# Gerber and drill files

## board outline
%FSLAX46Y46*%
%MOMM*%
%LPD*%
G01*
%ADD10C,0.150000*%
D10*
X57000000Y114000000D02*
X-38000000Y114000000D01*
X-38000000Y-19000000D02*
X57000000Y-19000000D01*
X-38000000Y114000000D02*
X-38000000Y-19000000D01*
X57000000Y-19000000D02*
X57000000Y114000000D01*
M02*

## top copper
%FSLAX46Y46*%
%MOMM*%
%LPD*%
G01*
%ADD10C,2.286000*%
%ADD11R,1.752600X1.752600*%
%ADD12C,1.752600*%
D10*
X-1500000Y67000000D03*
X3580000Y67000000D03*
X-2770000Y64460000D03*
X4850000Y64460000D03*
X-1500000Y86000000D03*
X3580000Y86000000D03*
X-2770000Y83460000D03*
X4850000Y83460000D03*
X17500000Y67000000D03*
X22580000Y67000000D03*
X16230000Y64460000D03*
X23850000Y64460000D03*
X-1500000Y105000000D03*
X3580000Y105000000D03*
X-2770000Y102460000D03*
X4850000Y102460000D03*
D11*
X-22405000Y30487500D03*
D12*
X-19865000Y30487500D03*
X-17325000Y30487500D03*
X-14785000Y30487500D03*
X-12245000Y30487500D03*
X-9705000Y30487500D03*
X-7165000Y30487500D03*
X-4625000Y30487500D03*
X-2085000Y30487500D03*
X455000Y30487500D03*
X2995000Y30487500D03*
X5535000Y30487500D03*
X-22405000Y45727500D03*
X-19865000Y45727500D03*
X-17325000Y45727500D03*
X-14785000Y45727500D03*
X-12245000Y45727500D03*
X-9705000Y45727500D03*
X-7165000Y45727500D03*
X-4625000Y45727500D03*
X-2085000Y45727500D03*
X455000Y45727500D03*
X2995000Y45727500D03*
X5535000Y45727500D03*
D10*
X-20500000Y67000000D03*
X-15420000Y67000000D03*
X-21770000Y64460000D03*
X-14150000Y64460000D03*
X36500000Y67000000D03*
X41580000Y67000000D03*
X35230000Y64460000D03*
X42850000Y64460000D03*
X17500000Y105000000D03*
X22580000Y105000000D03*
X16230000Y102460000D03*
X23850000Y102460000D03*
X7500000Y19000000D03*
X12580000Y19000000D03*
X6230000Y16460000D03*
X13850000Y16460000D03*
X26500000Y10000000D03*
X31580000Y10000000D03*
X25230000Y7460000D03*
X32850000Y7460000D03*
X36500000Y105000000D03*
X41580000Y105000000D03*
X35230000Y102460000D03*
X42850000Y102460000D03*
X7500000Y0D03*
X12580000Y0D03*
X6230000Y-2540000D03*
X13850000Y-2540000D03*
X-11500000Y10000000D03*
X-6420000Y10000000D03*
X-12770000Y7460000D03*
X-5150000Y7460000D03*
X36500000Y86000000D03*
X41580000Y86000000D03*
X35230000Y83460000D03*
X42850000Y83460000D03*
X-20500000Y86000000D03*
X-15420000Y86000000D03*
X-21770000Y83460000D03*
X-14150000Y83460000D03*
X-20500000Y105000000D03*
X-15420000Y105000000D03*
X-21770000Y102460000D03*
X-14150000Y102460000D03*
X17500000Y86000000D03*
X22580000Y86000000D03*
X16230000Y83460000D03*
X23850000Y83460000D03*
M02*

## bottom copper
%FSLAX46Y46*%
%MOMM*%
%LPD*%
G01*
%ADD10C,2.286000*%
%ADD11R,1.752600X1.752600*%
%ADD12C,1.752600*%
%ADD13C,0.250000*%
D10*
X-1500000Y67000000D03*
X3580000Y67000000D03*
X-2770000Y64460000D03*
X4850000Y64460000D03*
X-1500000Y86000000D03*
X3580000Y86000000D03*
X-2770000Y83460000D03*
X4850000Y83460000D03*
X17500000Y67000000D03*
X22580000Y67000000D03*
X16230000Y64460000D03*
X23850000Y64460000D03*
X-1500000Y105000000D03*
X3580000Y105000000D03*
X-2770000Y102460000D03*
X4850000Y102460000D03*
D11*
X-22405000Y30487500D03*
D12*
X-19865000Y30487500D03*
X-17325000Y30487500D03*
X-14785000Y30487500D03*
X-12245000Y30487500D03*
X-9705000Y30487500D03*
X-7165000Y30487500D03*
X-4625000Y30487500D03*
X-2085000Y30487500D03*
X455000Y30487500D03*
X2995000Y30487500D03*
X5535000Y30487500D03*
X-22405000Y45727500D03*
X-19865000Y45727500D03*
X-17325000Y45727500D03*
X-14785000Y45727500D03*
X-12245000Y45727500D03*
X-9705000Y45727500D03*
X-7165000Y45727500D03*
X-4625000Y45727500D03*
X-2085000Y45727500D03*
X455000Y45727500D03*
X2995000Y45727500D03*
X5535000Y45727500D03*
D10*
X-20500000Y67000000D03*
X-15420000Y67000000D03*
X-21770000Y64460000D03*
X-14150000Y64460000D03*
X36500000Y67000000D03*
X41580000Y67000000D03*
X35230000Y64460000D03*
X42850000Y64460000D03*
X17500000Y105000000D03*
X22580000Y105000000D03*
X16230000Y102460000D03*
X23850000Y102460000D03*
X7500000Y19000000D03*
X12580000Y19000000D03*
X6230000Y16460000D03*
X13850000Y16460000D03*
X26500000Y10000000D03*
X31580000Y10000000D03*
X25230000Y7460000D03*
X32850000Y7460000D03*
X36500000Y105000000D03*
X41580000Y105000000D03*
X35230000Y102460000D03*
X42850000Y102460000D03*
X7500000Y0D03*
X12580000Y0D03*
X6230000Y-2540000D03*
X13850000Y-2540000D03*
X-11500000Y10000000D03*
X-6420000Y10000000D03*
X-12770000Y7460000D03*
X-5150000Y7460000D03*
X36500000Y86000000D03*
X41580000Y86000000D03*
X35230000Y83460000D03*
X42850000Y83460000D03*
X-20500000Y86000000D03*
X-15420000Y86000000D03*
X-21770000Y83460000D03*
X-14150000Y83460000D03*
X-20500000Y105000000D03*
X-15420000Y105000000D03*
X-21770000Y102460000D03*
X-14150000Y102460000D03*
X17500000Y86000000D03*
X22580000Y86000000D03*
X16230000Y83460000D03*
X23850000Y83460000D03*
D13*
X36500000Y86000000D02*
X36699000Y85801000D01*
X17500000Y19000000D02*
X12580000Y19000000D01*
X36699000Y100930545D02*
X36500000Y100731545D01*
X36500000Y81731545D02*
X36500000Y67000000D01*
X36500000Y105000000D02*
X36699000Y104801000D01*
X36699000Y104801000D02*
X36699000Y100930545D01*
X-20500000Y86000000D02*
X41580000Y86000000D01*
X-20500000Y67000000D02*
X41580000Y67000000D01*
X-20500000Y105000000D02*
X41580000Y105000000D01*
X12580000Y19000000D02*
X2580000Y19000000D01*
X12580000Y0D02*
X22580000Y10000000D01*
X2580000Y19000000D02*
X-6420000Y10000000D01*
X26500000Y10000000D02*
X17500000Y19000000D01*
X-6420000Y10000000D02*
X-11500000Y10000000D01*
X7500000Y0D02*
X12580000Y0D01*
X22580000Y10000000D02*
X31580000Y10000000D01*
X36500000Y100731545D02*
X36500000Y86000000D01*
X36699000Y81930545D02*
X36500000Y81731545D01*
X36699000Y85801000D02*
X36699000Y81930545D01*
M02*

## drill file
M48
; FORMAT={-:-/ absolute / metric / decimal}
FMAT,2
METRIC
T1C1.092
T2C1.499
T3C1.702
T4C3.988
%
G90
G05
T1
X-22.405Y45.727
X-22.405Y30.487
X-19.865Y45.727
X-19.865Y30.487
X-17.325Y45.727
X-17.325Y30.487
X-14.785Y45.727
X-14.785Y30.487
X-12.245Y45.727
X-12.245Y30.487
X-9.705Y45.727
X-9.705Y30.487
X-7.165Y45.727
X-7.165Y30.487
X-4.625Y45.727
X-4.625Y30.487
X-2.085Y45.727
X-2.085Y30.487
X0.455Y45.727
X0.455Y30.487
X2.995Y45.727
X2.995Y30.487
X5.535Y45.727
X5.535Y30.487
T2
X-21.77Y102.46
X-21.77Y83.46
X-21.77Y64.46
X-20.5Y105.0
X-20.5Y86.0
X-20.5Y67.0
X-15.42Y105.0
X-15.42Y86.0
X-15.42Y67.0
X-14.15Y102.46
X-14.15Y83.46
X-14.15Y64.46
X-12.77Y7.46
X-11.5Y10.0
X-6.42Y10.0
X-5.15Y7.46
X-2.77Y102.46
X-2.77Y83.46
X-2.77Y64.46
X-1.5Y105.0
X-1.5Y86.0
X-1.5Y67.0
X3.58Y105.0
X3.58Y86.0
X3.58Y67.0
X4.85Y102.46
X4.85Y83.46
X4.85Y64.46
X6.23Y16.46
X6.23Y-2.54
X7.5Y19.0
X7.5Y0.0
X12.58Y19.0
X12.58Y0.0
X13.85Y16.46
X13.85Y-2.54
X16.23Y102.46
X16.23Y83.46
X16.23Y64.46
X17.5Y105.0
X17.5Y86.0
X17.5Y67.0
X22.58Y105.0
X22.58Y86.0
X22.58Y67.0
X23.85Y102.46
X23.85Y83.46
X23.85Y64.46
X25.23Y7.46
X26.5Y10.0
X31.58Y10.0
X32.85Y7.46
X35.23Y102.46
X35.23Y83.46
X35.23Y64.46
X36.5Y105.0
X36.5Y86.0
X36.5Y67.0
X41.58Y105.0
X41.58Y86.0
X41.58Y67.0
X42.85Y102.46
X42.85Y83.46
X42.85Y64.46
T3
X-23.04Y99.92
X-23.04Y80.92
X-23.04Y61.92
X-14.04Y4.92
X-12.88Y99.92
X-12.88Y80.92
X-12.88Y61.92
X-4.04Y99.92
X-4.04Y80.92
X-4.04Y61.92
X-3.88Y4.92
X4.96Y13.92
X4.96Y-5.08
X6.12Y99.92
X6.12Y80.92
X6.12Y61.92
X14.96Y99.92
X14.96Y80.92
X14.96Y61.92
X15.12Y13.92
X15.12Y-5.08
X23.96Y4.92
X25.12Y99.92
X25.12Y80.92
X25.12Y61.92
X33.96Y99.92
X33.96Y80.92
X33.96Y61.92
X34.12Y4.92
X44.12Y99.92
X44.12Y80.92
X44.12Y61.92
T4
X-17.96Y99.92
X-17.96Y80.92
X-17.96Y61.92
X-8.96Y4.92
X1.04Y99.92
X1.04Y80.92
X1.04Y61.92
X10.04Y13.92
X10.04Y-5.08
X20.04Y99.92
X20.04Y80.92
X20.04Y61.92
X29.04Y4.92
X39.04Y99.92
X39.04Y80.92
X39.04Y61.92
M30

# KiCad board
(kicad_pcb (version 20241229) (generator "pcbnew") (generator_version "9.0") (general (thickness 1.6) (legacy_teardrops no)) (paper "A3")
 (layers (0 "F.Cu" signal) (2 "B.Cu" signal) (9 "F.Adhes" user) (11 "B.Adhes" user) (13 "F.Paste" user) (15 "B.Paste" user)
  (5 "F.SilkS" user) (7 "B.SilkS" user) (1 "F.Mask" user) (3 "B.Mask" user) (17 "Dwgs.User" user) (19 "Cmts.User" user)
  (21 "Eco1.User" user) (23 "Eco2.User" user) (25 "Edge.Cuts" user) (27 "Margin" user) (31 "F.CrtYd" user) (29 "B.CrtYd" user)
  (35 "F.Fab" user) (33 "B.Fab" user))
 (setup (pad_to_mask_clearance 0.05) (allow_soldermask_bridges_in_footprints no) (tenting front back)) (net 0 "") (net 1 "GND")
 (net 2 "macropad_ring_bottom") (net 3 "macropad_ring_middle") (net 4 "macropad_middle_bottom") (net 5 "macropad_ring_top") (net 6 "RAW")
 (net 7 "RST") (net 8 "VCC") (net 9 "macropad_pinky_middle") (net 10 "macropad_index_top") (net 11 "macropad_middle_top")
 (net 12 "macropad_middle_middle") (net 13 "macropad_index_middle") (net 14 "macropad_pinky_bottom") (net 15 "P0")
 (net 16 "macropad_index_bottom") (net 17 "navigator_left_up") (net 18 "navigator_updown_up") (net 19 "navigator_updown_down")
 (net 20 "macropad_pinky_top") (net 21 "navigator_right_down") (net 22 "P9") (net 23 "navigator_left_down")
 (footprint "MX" (layer "F.Cu") (at 1.04 -61.92)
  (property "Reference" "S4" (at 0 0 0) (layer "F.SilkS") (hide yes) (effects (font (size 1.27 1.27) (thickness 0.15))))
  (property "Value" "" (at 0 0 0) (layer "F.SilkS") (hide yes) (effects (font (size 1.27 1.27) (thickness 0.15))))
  (pad "" np_thru_hole circle (at -5.08 0) (size 1.7018 1.7018) (drill 1.7018) (layers "*.Cu" "*.Mask"))
  (pad "" np_thru_hole circle (at 0 0) (size 3.9878 3.9878) (drill 3.9878) (layers "*.Cu" "*.Mask"))
  (pad "" np_thru_hole circle (at 5.08 0) (size 1.7018 1.7018) (drill 1.7018) (layers "*.Cu" "*.Mask"))
  (pad "1" thru_hole circle (at -2.54 -5.08) (size 2.286 2.286) (drill 1.4986) (layers "*.Cu" "*.Mask") (remove_unused_layers no)
   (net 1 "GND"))
  (pad "1" thru_hole circle (at 2.54 -5.08) (size 2.286 2.286) (drill 1.4986) (layers "*.Cu" "*.Mask") (remove_unused_layers no)
   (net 1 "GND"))
  (pad "2" thru_hole circle (at -3.81 -2.54) (size 2.286 2.286) (drill 1.4986) (layers "*.Cu" "*.Mask") (remove_unused_layers no)
   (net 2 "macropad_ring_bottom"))
  (pad "2" thru_hole circle (at 3.81 -2.54) (size 2.286 2.286) (drill 1.4986) (layers "*.Cu" "*.Mask") (remove_unused_layers no)
   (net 2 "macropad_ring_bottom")))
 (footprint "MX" (layer "F.Cu") (at 1.04 -80.92)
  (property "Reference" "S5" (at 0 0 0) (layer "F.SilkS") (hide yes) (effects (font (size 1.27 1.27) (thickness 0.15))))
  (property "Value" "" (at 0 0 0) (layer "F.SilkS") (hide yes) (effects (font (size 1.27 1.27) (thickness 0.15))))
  (pad "" np_thru_hole circle (at -5.08 0) (size 1.7018 1.7018) (drill 1.7018) (layers "*.Cu" "*.Mask"))
  (pad "" np_thru_hole circle (at 0 0) (size 3.9878 3.9878) (drill 3.9878) (layers "*.Cu" "*.Mask"))
  (pad "" np_thru_hole circle (at 5.08 0) (size 1.7018 1.7018) (drill 1.7018) (layers "*.Cu" "*.Mask"))
  (pad "1" thru_hole circle (at -2.54 -5.08) (size 2.286 2.286) (drill 1.4986) (layers "*.Cu" "*.Mask") (remove_unused_layers no)
   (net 1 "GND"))
  (pad "1" thru_hole circle (at 2.54 -5.08) (size 2.286 2.286) (drill 1.4986) (layers "*.Cu" "*.Mask") (remove_unused_layers no)
   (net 1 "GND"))
  (pad "2" thru_hole circle (at -3.81 -2.54) (size 2.286 2.286) (drill 1.4986) (layers "*.Cu" "*.Mask") (remove_unused_layers no)
   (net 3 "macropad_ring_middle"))
  (pad "2" thru_hole circle (at 3.81 -2.54) (size 2.286 2.286) (drill 1.4986) (layers "*.Cu" "*.Mask") (remove_unused_layers no)
   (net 3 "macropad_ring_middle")))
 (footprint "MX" (layer "F.Cu") (at 20.04 -61.92)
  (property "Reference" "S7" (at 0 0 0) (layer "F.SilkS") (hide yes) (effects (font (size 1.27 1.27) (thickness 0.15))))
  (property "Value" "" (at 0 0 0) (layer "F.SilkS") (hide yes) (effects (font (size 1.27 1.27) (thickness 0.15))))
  (pad "" np_thru_hole circle (at -5.08 0) (size 1.7018 1.7018) (drill 1.7018) (layers "*.Cu" "*.Mask"))
  (pad "" np_thru_hole circle (at 0 0) (size 3.9878 3.9878) (drill 3.9878) (layers "*.Cu" "*.Mask"))
  (pad "" np_thru_hole circle (at 5.08 0) (size 1.7018 1.7018) (drill 1.7018) (layers "*.Cu" "*.Mask"))
  (pad "1" thru_hole circle (at -2.54 -5.08) (size 2.286 2.286) (drill 1.4986) (layers "*.Cu" "*.Mask") (remove_unused_layers no)
   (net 1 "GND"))
  (pad "1" thru_hole circle (at 2.54 -5.08) (size 2.286 2.286) (drill 1.4986) (layers "*.Cu" "*.Mask") (remove_unused_layers no)
   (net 1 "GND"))
  (pad "2" thru_hole circle (at -3.81 -2.54) (size 2.286 2.286) (drill 1.4986) (layers "*.Cu" "*.Mask") (remove_unused_layers no)
   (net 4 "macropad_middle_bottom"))
  (pad "2" thru_hole circle (at 3.81 -2.54) (size 2.286 2.286) (drill 1.4986) (layers "*.Cu" "*.Mask") (remove_unused_layers no)
   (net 4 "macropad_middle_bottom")))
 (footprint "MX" (layer "F.Cu") (at 1.04 -99.92)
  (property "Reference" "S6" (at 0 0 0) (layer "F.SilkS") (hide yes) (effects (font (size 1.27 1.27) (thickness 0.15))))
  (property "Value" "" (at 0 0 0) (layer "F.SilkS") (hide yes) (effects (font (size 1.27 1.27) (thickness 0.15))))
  (pad "" np_thru_hole circle (at -5.08 0) (size 1.7018 1.7018) (drill 1.7018) (layers "*.Cu" "*.Mask"))
  (pad "" np_thru_hole circle (at 0 0) (size 3.9878 3.9878) (drill 3.9878) (layers "*.Cu" "*.Mask"))
  (pad "" np_thru_hole circle (at 5.08 0) (size 1.7018 1.7018) (drill 1.7018) (layers "*.Cu" "*.Mask"))
  (pad "1" thru_hole circle (at -2.54 -5.08) (size 2.286 2.286) (drill 1.4986) (layers "*.Cu" "*.Mask") (remove_unused_layers no)
   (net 1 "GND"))
  (pad "1" thru_hole circle (at 2.54 -5.08) (size 2.286 2.286) (drill 1.4986) (layers "*.Cu" "*.Mask") (remove_unused_layers no)
   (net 1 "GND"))
  (pad "2" thru_hole circle (at -3.81 -2.54) (size 2.286 2.286) (drill 1.4986) (layers "*.Cu" "*.Mask") (remove_unused_layers no)
   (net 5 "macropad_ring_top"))
  (pad "2" thru_hole circle (at 3.81 -2.54) (size 2.286 2.286) (drill 1.4986) (layers "*.Cu" "*.Mask") (remove_unused_layers no)
   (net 5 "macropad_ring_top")))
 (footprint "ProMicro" (layer "F.Cu") (at -8.435 -38.1075)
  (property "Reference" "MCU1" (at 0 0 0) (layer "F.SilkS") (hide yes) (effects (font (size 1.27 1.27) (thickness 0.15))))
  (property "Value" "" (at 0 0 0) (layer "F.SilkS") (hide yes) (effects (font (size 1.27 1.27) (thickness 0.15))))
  (pad "1" thru_hole rect (at -13.97 7.62) (size 1.7526 1.7526) (drill 1.0922) (layers "*.Cu" "*.SilkS" "*.Mask") (remove_unused_layers no)
   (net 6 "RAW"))
  (pad "2" thru_hole circle (at -11.43 7.62) (size 1.7526 1.7526) (drill 1.0922) (layers "*.Cu" "*.SilkS" "*.Mask")
   (remove_unused_layers no) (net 1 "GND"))
  (pad "3" thru_hole circle (at -8.89 7.62) (size 1.7526 1.7526) (drill 1.0922) (layers "*.Cu" "*.SilkS" "*.Mask") (remove_unused_layers no)
   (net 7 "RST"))
  (pad "4" thru_hole circle (at -6.35 7.62) (size 1.7526 1.7526) (drill 1.0922) (layers "*.Cu" "*.SilkS" "*.Mask") (remove_unused_layers no)
   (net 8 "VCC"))
  (pad "5" thru_hole circle (at -3.81 7.62) (size 1.7526 1.7526) (drill 1.0922) (layers "*.Cu" "*.SilkS" "*.Mask") (remove_unused_layers no)
   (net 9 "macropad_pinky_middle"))
  (pad "6" thru_hole circle (at -1.27 7.62) (size 1.7526 1.7526) (drill 1.0922) (layers "*.Cu" "*.SilkS" "*.Mask") (remove_unused_layers no)
   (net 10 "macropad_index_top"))
  (pad "7" thru_hole circle (at 1.27 7.62) (size 1.7526 1.7526) (drill 1.0922) (layers "*.Cu" "*.SilkS" "*.Mask") (remove_unused_layers no)
   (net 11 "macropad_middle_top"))
  (pad "8" thru_hole circle (at 3.81 7.62) (size 1.7526 1.7526) (drill 1.0922) (layers "*.Cu" "*.SilkS" "*.Mask") (remove_unused_layers no)
   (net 5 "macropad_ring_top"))
  (pad "9" thru_hole circle (at 6.35 7.62) (size 1.7526 1.7526) (drill 1.0922) (layers "*.Cu" "*.SilkS" "*.Mask") (remove_unused_layers no)
   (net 3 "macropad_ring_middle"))
  (pad "10" thru_hole circle (at 8.89 7.62) (size 1.7526 1.7526) (drill 1.0922) (layers "*.Cu" "*.SilkS" "*.Mask") (remove_unused_layers no)
   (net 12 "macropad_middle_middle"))
  (pad "11" thru_hole circle (at 11.43 7.62) (size 1.7526 1.7526) (drill 1.0922) (layers "*.Cu" "*.SilkS" "*.Mask")
   (remove_unused_layers no) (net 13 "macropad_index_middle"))
  (pad "12" thru_hole circle (at 13.97 7.62) (size 1.7526 1.7526) (drill 1.0922) (layers "*.Cu" "*.SilkS" "*.Mask")
   (remove_unused_layers no) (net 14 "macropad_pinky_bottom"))
  (pad "13" thru_hole circle (at -13.97 -7.62) (size 1.7526 1.7526) (drill 1.0922) (layers "*.Cu" "*.SilkS" "*.Mask")
   (remove_unused_layers no) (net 2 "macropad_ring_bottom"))
  (pad "14" thru_hole circle (at -11.43 -7.62) (size 1.7526 1.7526) (drill 1.0922) (layers "*.Cu" "*.SilkS" "*.Mask")
   (remove_unused_layers no) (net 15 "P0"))
  (pad "15" thru_hole circle (at -8.89 -7.62) (size 1.7526 1.7526) (drill 1.0922) (layers "*.Cu" "*.SilkS" "*.Mask")
   (remove_unused_layers no) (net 1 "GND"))
  (pad "16" thru_hole circle (at -6.35 -7.62) (size 1.7526 1.7526) (drill 1.0922) (layers "*.Cu" "*.SilkS" "*.Mask")
   (remove_unused_layers no) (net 1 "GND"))
  (pad "17" thru_hole circle (at -3.81 -7.62) (size 1.7526 1.7526) (drill 1.0922) (layers "*.Cu" "*.SilkS" "*.Mask")
   (remove_unused_layers no) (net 4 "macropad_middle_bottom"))
  (pad "18" thru_hole circle (at -1.27 -7.62) (size 1.7526 1.7526) (drill 1.0922) (layers "*.Cu" "*.SilkS" "*.Mask")
   (remove_unused_layers no) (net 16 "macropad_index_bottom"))
  (pad "19" thru_hole circle (at 1.27 -7.62) (size 1.7526 1.7526) (drill 1.0922) (layers "*.Cu" "*.SilkS" "*.Mask")
   (remove_unused_layers no) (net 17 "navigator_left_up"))
  (pad "20" thru_hole circle (at 3.81 -7.62) (size 1.7526 1.7526) (drill 1.0922) (layers "*.Cu" "*.SilkS" "*.Mask")
   (remove_unused_layers no) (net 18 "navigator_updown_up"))
  (pad "21" thru_hole circle (at 6.35 -7.62) (size 1.7526 1.7526) (drill 1.0922) (layers "*.Cu" "*.SilkS" "*.Mask")
   (remove_unused_layers no) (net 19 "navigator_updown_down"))
  (pad "22" thru_hole circle (at 8.89 -7.62) (size 1.7526 1.7526) (drill 1.0922) (layers "*.Cu" "*.SilkS" "*.Mask")
   (remove_unused_layers no) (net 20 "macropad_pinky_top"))
  (pad "23" thru_hole circle (at 11.43 -7.62) (size 1.7526 1.7526) (drill 1.0922) (layers "*.Cu" "*.SilkS" "*.Mask")
   (remove_unused_layers no) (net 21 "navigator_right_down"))
  (pad "24" thru_hole circle (at 13.97 -7.62) (size 1.7526 1.7526) (drill 1.0922) (layers "*.Cu" "*.SilkS" "*.Mask")
   (remove_unused_layers no) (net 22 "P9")))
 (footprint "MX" (layer "F.Cu") (at -17.96 -61.92)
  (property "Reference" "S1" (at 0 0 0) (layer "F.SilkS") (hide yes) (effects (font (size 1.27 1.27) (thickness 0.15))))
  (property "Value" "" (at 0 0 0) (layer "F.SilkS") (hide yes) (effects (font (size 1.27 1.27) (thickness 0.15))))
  (pad "" np_thru_hole circle (at -5.08 0) (size 1.7018 1.7018) (drill 1.7018) (layers "*.Cu" "*.Mask"))
  (pad "" np_thru_hole circle (at 0 0) (size 3.9878 3.9878) (drill 3.9878) (layers "*.Cu" "*.Mask"))
  (pad "" np_thru_hole circle (at 5.08 0) (size 1.7018 1.7018) (drill 1.7018) (layers "*.Cu" "*.Mask"))
  (pad "1" thru_hole circle (at -2.54 -5.08) (size 2.286 2.286) (drill 1.4986) (layers "*.Cu" "*.Mask") (remove_unused_layers no)
   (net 1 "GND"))
  (pad "1" thru_hole circle (at 2.54 -5.08) (size 2.286 2.286) (drill 1.4986) (layers "*.Cu" "*.Mask") (remove_unused_layers no)
   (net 1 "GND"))
  (pad "2" thru_hole circle (at -3.81 -2.54) (size 2.286 2.286) (drill 1.4986) (layers "*.Cu" "*.Mask") (remove_unused_layers no)
   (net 14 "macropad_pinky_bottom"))
  (pad "2" thru_hole circle (at 3.81 -2.54) (size 2.286 2.286) (drill 1.4986) (layers "*.Cu" "*.Mask") (remove_unused_layers no)
   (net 14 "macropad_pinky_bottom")))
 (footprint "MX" (layer "F.Cu") (at 39.04 -61.92)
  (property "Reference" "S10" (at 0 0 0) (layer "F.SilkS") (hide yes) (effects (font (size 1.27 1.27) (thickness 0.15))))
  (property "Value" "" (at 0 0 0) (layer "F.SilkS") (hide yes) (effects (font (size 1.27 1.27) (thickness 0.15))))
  (pad "" np_thru_hole circle (at -5.08 0) (size 1.7018 1.7018) (drill 1.7018) (layers "*.Cu" "*.Mask"))
  (pad "" np_thru_hole circle (at 0 0) (size 3.9878 3.9878) (drill 3.9878) (layers "*.Cu" "*.Mask"))
  (pad "" np_thru_hole circle (at 5.08 0) (size 1.7018 1.7018) (drill 1.7018) (layers "*.Cu" "*.Mask"))
  (pad "1" thru_hole circle (at -2.54 -5.08) (size 2.286 2.286) (drill 1.4986) (layers "*.Cu" "*.Mask") (remove_unused_layers no)
   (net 1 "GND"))
  (pad "1" thru_hole circle (at 2.54 -5.08) (size 2.286 2.286) (drill 1.4986) (layers "*.Cu" "*.Mask") (remove_unused_layers no)
   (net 1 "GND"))
  (pad "2" thru_hole circle (at -3.81 -2.54) (size 2.286 2.286) (drill 1.4986) (layers "*.Cu" "*.Mask") (remove_unused_layers no)
   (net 16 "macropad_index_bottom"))
  (pad "2" thru_hole circle (at 3.81 -2.54) (size 2.286 2.286) (drill 1.4986) (layers "*.Cu" "*.Mask") (remove_unused_layers no)
   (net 16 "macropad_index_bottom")))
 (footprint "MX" (layer "F.Cu") (at 20.04 -99.92)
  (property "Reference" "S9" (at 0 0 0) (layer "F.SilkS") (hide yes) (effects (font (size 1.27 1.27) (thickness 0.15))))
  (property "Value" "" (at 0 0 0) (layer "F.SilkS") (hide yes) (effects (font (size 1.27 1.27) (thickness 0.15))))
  (pad "" np_thru_hole circle (at -5.08 0) (size 1.7018 1.7018) (drill 1.7018) (layers "*.Cu" "*.Mask"))
  (pad "" np_thru_hole circle (at 0 0) (size 3.9878 3.9878) (drill 3.9878) (layers "*.Cu" "*.Mask"))
  (pad "" np_thru_hole circle (at 5.08 0) (size 1.7018 1.7018) (drill 1.7018) (layers "*.Cu" "*.Mask"))
  (pad "1" thru_hole circle (at -2.54 -5.08) (size 2.286 2.286) (drill 1.4986) (layers "*.Cu" "*.Mask") (remove_unused_layers no)
   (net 1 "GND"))
  (pad "1" thru_hole circle (at 2.54 -5.08) (size 2.286 2.286) (drill 1.4986) (layers "*.Cu" "*.Mask") (remove_unused_layers no)
   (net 1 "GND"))
  (pad "2" thru_hole circle (at -3.81 -2.54) (size 2.286 2.286) (drill 1.4986) (layers "*.Cu" "*.Mask") (remove_unused_layers no)
   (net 11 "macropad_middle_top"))
  (pad "2" thru_hole circle (at 3.81 -2.54) (size 2.286 2.286) (drill 1.4986) (layers "*.Cu" "*.Mask") (remove_unused_layers no)
   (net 11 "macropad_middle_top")))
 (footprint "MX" (layer "F.Cu") (at 10.04 -13.92)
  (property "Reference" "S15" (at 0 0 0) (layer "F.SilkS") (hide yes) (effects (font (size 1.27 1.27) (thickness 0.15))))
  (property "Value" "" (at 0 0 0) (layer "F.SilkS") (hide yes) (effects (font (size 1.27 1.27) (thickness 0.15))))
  (pad "" np_thru_hole circle (at -5.08 0) (size 1.7018 1.7018) (drill 1.7018) (layers "*.Cu" "*.Mask"))
  (pad "" np_thru_hole circle (at 0 0) (size 3.9878 3.9878) (drill 3.9878) (layers "*.Cu" "*.Mask"))
  (pad "" np_thru_hole circle (at 5.08 0) (size 1.7018 1.7018) (drill 1.7018) (layers "*.Cu" "*.Mask"))
  (pad "1" thru_hole circle (at -2.54 -5.08) (size 2.286 2.286) (drill 1.4986) (layers "*.Cu" "*.Mask") (remove_unused_layers no)
   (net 1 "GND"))
  (pad "1" thru_hole circle (at 2.54 -5.08) (size 2.286 2.286) (drill 1.4986) (layers "*.Cu" "*.Mask") (remove_unused_layers no)
   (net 1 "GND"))
  (pad "2" thru_hole circle (at -3.81 -2.54) (size 2.286 2.286) (drill 1.4986) (layers "*.Cu" "*.Mask") (remove_unused_layers no)
   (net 18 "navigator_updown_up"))
  (pad "2" thru_hole circle (at 3.81 -2.54) (size 2.286 2.286) (drill 1.4986) (layers "*.Cu" "*.Mask") (remove_unused_layers no)
   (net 18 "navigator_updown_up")))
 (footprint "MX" (layer "F.Cu") (at 29.04 -4.92)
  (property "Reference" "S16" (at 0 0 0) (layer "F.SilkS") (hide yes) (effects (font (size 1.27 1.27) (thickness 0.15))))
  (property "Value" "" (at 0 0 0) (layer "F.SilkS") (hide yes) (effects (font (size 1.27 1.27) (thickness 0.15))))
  (pad "" np_thru_hole circle (at -5.08 0) (size 1.7018 1.7018) (drill 1.7018) (layers "*.Cu" "*.Mask"))
  (pad "" np_thru_hole circle (at 0 0) (size 3.9878 3.9878) (drill 3.9878) (layers "*.Cu" "*.Mask"))
  (pad "" np_thru_hole circle (at 5.08 0) (size 1.7018 1.7018) (drill 1.7018) (layers "*.Cu" "*.Mask"))
  (pad "1" thru_hole circle (at -2.54 -5.08) (size 2.286 2.286) (drill 1.4986) (layers "*.Cu" "*.Mask") (remove_unused_layers no)
   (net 1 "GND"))
  (pad "1" thru_hole circle (at 2.54 -5.08) (size 2.286 2.286) (drill 1.4986) (layers "*.Cu" "*.Mask") (remove_unused_layers no)
   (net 1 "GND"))
  (pad "2" thru_hole circle (at -3.81 -2.54) (size 2.286 2.286) (drill 1.4986) (layers "*.Cu" "*.Mask") (remove_unused_layers no)
   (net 21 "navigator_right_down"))
  (pad "2" thru_hole circle (at 3.81 -2.54) (size 2.286 2.286) (drill 1.4986) (layers "*.Cu" "*.Mask") (remove_unused_layers no)
   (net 21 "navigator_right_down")))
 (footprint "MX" (layer "F.Cu") (at 39.04 -99.92)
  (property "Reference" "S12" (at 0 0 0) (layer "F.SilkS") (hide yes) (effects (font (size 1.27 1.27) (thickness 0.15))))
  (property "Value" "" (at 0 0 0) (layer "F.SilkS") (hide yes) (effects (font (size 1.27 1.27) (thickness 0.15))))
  (pad "" np_thru_hole circle (at -5.08 0) (size 1.7018 1.7018) (drill 1.7018) (layers "*.Cu" "*.Mask"))
  (pad "" np_thru_hole circle (at 0 0) (size 3.9878 3.9878) (drill 3.9878) (layers "*.Cu" "*.Mask"))
  (pad "" np_thru_hole circle (at 5.08 0) (size 1.7018 1.7018) (drill 1.7018) (layers "*.Cu" "*.Mask"))
  (pad "1" thru_hole circle (at -2.54 -5.08) (size 2.286 2.286) (drill 1.4986) (layers "*.Cu" "*.Mask") (remove_unused_layers no)
   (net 1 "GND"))
  (pad "1" thru_hole circle (at 2.54 -5.08) (size 2.286 2.286) (drill 1.4986) (layers "*.Cu" "*.Mask") (remove_unused_layers no)
   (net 1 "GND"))
  (pad "2" thru_hole circle (at -3.81 -2.54) (size 2.286 2.286) (drill 1.4986) (layers "*.Cu" "*.Mask") (remove_unused_layers no)
   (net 10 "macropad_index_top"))
  (pad "2" thru_hole circle (at 3.81 -2.54) (size 2.286 2.286) (drill 1.4986) (layers "*.Cu" "*.Mask") (remove_unused_layers no)
   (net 10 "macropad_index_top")))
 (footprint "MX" (layer "F.Cu") (at 10.04 5.08)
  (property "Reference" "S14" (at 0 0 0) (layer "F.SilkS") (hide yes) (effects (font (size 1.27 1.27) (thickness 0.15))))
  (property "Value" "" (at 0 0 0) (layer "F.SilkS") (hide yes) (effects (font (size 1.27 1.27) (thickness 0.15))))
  (pad "" np_thru_hole circle (at -5.08 0) (size 1.7018 1.7018) (drill 1.7018) (layers "*.Cu" "*.Mask"))
  (pad "" np_thru_hole circle (at 0 0) (size 3.9878 3.9878) (drill 3.9878) (layers "*.Cu" "*.Mask"))
  (pad "" np_thru_hole circle (at 5.08 0) (size 1.7018 1.7018) (drill 1.7018) (layers "*.Cu" "*.Mask"))
  (pad "1" thru_hole circle (at -2.54 -5.08) (size 2.286 2.286) (drill 1.4986) (layers "*.Cu" "*.Mask") (remove_unused_layers no)
   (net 1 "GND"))
  (pad "1" thru_hole circle (at 2.54 -5.08) (size 2.286 2.286) (drill 1.4986) (layers "*.Cu" "*.Mask") (remove_unused_layers no)
   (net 1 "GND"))
  (pad "2" thru_hole circle (at -3.81 -2.54) (size 2.286 2.286) (drill 1.4986) (layers "*.Cu" "*.Mask") (remove_unused_layers no)
   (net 19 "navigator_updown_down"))
  (pad "2" thru_hole circle (at 3.81 -2.54) (size 2.286 2.286) (drill 1.4986) (layers "*.Cu" "*.Mask") (remove_unused_layers no)
   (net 19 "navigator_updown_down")))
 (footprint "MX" (layer "F.Cu") (at -8.96 -4.92)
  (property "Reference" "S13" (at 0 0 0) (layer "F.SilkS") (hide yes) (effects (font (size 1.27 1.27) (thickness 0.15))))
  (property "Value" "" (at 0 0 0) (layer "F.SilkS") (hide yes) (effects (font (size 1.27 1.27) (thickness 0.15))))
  (pad "" np_thru_hole circle (at -5.08 0) (size 1.7018 1.7018) (drill 1.7018) (layers "*.Cu" "*.Mask"))
  (pad "" np_thru_hole circle (at 0 0) (size 3.9878 3.9878) (drill 3.9878) (layers "*.Cu" "*.Mask"))
  (pad "" np_thru_hole circle (at 5.08 0) (size 1.7018 1.7018) (drill 1.7018) (layers "*.Cu" "*.Mask"))
  (pad "1" thru_hole circle (at -2.54 -5.08) (size 2.286 2.286) (drill 1.4986) (layers "*.Cu" "*.Mask") (remove_unused_layers no)
   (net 1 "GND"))
  (pad "1" thru_hole circle (at 2.54 -5.08) (size 2.286 2.286) (drill 1.4986) (layers "*.Cu" "*.Mask") (remove_unused_layers no)
   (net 1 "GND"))
  (pad "2" thru_hole circle (at -3.81 -2.54) (size 2.286 2.286) (drill 1.4986) (layers "*.Cu" "*.Mask") (remove_unused_layers no)
   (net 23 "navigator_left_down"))
  (pad "2" thru_hole circle (at 3.81 -2.54) (size 2.286 2.286) (drill 1.4986) (layers "*.Cu" "*.Mask") (remove_unused_layers no)
   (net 23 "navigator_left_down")))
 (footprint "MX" (layer "F.Cu") (at 39.04 -80.92)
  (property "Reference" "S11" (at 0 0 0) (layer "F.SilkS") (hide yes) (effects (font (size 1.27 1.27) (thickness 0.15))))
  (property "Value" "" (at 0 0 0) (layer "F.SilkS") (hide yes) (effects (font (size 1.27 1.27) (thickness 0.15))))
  (pad "" np_thru_hole circle (at -5.08 0) (size 1.7018 1.7018) (drill 1.7018) (layers "*.Cu" "*.Mask"))
  (pad "" np_thru_hole circle (at 0 0) (size 3.9878 3.9878) (drill 3.9878) (layers "*.Cu" "*.Mask"))
  (pad "" np_thru_hole circle (at 5.08 0) (size 1.7018 1.7018) (drill 1.7018) (layers "*.Cu" "*.Mask"))
  (pad "1" thru_hole circle (at -2.54 -5.08) (size 2.286 2.286) (drill 1.4986) (layers "*.Cu" "*.Mask") (remove_unused_layers no)
   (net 1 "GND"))
  (pad "1" thru_hole circle (at 2.54 -5.08) (size 2.286 2.286) (drill 1.4986) (layers "*.Cu" "*.Mask") (remove_unused_layers no)
   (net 1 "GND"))
  (pad "2" thru_hole circle (at -3.81 -2.54) (size 2.286 2.286) (drill 1.4986) (layers "*.Cu" "*.Mask") (remove_unused_layers no)
   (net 13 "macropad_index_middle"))
  (pad "2" thru_hole circle (at 3.81 -2.54) (size 2.286 2.286) (drill 1.4986) (layers "*.Cu" "*.Mask") (remove_unused_layers no)
   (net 13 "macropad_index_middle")))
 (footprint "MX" (layer "F.Cu") (at -17.96 -80.92)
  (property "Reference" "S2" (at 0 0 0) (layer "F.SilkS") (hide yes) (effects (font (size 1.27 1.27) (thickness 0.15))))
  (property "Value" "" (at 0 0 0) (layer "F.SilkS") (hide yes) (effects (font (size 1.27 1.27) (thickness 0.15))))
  (pad "" np_thru_hole circle (at -5.08 0) (size 1.7018 1.7018) (drill 1.7018) (layers "*.Cu" "*.Mask"))
  (pad "" np_thru_hole circle (at 0 0) (size 3.9878 3.9878) (drill 3.9878) (layers "*.Cu" "*.Mask"))
  (pad "" np_thru_hole circle (at 5.08 0) (size 1.7018 1.7018) (drill 1.7018) (layers "*.Cu" "*.Mask"))
  (pad "1" thru_hole circle (at -2.54 -5.08) (size 2.286 2.286) (drill 1.4986) (layers "*.Cu" "*.Mask") (remove_unused_layers no)
   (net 1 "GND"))
  (pad "1" thru_hole circle (at 2.54 -5.08) (size 2.286 2.286) (drill 1.4986) (layers "*.Cu" "*.Mask") (remove_unused_layers no)
   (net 1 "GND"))
  (pad "2" thru_hole circle (at -3.81 -2.54) (size 2.286 2.286) (drill 1.4986) (layers "*.Cu" "*.Mask") (remove_unused_layers no)
   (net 9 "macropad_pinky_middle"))
  (pad "2" thru_hole circle (at 3.81 -2.54) (size 2.286 2.286) (drill 1.4986) (layers "*.Cu" "*.Mask") (remove_unused_layers no)
   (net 9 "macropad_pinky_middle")))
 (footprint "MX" (layer "F.Cu") (at -17.96 -99.92)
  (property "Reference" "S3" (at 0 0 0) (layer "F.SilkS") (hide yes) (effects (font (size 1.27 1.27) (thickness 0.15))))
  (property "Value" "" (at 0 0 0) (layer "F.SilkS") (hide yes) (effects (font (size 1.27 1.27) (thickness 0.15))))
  (pad "" np_thru_hole circle (at -5.08 0) (size 1.7018 1.7018) (drill 1.7018) (layers "*.Cu" "*.Mask"))
  (pad "" np_thru_hole circle (at 0 0) (size 3.9878 3.9878) (drill 3.9878) (layers "*.Cu" "*.Mask"))
  (pad "" np_thru_hole circle (at 5.08 0) (size 1.7018 1.7018) (drill 1.7018) (layers "*.Cu" "*.Mask"))
  (pad "1" thru_hole circle (at -2.54 -5.08) (size 2.286 2.286) (drill 1.4986) (layers "*.Cu" "*.Mask") (remove_unused_layers no)
   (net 1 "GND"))
  (pad "1" thru_hole circle (at 2.54 -5.08) (size 2.286 2.286) (drill 1.4986) (layers "*.Cu" "*.Mask") (remove_unused_layers no)
   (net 1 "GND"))
  (pad "2" thru_hole circle (at -3.81 -2.54) (size 2.286 2.286) (drill 1.4986) (layers "*.Cu" "*.Mask") (remove_unused_layers no)
   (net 20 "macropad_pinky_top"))
  (pad "2" thru_hole circle (at 3.81 -2.54) (size 2.286 2.286) (drill 1.4986) (layers "*.Cu" "*.Mask") (remove_unused_layers no)
   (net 20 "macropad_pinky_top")))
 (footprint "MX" (layer "F.Cu") (at 20.04 -80.92)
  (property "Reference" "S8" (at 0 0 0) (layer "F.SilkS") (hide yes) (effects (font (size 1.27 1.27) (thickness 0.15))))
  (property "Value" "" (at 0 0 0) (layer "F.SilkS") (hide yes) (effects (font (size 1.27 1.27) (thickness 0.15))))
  (pad "" np_thru_hole circle (at -5.08 0) (size 1.7018 1.7018) (drill 1.7018) (layers "*.Cu" "*.Mask"))
  (pad "" np_thru_hole circle (at 0 0) (size 3.9878 3.9878) (drill 3.9878) (layers "*.Cu" "*.Mask"))
  (pad "" np_thru_hole circle (at 5.08 0) (size 1.7018 1.7018) (drill 1.7018) (layers "*.Cu" "*.Mask"))
  (pad "1" thru_hole circle (at -2.54 -5.08) (size 2.286 2.286) (drill 1.4986) (layers "*.Cu" "*.Mask") (remove_unused_layers no)
   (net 1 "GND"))
  (pad "1" thru_hole circle (at 2.54 -5.08) (size 2.286 2.286) (drill 1.4986) (layers "*.Cu" "*.Mask") (remove_unused_layers no)
   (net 1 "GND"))
  (pad "2" thru_hole circle (at -3.81 -2.54) (size 2.286 2.286) (drill 1.4986) (layers "*.Cu" "*.Mask") (remove_unused_layers no)
   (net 12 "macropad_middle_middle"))
  (pad "2" thru_hole circle (at 3.81 -2.54) (size 2.286 2.286) (drill 1.4986) (layers "*.Cu" "*.Mask") (remove_unused_layers no)
   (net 12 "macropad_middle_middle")))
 (gr_line (start 57 -114) (end -38 -114) (stroke (width 0.15) (type solid)) (layer "Edge.Cuts"))
 (gr_line (start -38 19) (end 57 19) (stroke (width 0.15) (type solid)) (layer "Edge.Cuts"))
 (gr_line (start -38 -114) (end -38 19) (stroke (width 0.15) (type solid)) (layer "Edge.Cuts"))
 (gr_line (start 57 19) (end 57 -114) (stroke (width 0.15) (type solid)) (layer "Edge.Cuts"))
 (segment (start 36.5 -86) (end 36.699 -85.801) (width 0.25) (layer "B.Cu") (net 1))
 (segment (start 17.5 -19) (end 12.58 -19) (width 0.25) (layer "B.Cu") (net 1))
 (segment (start 36.699 -100.930545) (end 36.5 -100.731545) (width 0.25) (layer "B.Cu") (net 1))
 (segment (start 36.5 -81.731545) (end 36.5 -67) (width 0.25) (layer "B.Cu") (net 1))
 (segment (start 36.5 -105) (end 36.699 -104.801) (width 0.25) (layer "B.Cu") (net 1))
 (segment (start 36.699 -104.801) (end 36.699 -100.930545) (width 0.25) (layer "B.Cu") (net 1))
 (segment (start -20.5 -86) (end 41.58 -86) (width 0.25) (layer "B.Cu") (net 1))
 (segment (start -20.5 -67) (end 41.58 -67) (width 0.25) (layer "B.Cu") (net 1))
 (segment (start -20.5 -105) (end 41.58 -105) (width 0.25) (layer "B.Cu") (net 1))
 (segment (start 12.58 -19) (end 2.58 -19) (width 0.25) (layer "B.Cu") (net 1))
 (segment (start 12.58 0) (end 22.58 -10) (width 0.25) (layer "B.Cu") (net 1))
 (segment (start 2.58 -19) (end -6.42 -10) (width 0.25) (layer "B.Cu") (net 1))
 (segment (start 26.5 -10) (end 17.5 -19) (width 0.25) (layer "B.Cu") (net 1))
 (segment (start -6.42 -10) (end -11.5 -10) (width 0.25) (layer "B.Cu") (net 1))
 (segment (start 7.5 0) (end 12.58 0) (width 0.25) (layer "B.Cu") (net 1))
 (segment (start 22.58 -10) (end 31.58 -10) (width 0.25) (layer "B.Cu") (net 1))
 (segment (start 36.5 -100.731545) (end 36.5 -86) (width 0.25) (layer "B.Cu") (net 1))
 (segment (start 36.699 -81.930545) (end 36.5 -81.731545) (width 0.25) (layer "B.Cu") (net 1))
 (segment (start 36.699 -85.801) (end 36.699 -81.930545) (width 0.25) (layer "B.Cu") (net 1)))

